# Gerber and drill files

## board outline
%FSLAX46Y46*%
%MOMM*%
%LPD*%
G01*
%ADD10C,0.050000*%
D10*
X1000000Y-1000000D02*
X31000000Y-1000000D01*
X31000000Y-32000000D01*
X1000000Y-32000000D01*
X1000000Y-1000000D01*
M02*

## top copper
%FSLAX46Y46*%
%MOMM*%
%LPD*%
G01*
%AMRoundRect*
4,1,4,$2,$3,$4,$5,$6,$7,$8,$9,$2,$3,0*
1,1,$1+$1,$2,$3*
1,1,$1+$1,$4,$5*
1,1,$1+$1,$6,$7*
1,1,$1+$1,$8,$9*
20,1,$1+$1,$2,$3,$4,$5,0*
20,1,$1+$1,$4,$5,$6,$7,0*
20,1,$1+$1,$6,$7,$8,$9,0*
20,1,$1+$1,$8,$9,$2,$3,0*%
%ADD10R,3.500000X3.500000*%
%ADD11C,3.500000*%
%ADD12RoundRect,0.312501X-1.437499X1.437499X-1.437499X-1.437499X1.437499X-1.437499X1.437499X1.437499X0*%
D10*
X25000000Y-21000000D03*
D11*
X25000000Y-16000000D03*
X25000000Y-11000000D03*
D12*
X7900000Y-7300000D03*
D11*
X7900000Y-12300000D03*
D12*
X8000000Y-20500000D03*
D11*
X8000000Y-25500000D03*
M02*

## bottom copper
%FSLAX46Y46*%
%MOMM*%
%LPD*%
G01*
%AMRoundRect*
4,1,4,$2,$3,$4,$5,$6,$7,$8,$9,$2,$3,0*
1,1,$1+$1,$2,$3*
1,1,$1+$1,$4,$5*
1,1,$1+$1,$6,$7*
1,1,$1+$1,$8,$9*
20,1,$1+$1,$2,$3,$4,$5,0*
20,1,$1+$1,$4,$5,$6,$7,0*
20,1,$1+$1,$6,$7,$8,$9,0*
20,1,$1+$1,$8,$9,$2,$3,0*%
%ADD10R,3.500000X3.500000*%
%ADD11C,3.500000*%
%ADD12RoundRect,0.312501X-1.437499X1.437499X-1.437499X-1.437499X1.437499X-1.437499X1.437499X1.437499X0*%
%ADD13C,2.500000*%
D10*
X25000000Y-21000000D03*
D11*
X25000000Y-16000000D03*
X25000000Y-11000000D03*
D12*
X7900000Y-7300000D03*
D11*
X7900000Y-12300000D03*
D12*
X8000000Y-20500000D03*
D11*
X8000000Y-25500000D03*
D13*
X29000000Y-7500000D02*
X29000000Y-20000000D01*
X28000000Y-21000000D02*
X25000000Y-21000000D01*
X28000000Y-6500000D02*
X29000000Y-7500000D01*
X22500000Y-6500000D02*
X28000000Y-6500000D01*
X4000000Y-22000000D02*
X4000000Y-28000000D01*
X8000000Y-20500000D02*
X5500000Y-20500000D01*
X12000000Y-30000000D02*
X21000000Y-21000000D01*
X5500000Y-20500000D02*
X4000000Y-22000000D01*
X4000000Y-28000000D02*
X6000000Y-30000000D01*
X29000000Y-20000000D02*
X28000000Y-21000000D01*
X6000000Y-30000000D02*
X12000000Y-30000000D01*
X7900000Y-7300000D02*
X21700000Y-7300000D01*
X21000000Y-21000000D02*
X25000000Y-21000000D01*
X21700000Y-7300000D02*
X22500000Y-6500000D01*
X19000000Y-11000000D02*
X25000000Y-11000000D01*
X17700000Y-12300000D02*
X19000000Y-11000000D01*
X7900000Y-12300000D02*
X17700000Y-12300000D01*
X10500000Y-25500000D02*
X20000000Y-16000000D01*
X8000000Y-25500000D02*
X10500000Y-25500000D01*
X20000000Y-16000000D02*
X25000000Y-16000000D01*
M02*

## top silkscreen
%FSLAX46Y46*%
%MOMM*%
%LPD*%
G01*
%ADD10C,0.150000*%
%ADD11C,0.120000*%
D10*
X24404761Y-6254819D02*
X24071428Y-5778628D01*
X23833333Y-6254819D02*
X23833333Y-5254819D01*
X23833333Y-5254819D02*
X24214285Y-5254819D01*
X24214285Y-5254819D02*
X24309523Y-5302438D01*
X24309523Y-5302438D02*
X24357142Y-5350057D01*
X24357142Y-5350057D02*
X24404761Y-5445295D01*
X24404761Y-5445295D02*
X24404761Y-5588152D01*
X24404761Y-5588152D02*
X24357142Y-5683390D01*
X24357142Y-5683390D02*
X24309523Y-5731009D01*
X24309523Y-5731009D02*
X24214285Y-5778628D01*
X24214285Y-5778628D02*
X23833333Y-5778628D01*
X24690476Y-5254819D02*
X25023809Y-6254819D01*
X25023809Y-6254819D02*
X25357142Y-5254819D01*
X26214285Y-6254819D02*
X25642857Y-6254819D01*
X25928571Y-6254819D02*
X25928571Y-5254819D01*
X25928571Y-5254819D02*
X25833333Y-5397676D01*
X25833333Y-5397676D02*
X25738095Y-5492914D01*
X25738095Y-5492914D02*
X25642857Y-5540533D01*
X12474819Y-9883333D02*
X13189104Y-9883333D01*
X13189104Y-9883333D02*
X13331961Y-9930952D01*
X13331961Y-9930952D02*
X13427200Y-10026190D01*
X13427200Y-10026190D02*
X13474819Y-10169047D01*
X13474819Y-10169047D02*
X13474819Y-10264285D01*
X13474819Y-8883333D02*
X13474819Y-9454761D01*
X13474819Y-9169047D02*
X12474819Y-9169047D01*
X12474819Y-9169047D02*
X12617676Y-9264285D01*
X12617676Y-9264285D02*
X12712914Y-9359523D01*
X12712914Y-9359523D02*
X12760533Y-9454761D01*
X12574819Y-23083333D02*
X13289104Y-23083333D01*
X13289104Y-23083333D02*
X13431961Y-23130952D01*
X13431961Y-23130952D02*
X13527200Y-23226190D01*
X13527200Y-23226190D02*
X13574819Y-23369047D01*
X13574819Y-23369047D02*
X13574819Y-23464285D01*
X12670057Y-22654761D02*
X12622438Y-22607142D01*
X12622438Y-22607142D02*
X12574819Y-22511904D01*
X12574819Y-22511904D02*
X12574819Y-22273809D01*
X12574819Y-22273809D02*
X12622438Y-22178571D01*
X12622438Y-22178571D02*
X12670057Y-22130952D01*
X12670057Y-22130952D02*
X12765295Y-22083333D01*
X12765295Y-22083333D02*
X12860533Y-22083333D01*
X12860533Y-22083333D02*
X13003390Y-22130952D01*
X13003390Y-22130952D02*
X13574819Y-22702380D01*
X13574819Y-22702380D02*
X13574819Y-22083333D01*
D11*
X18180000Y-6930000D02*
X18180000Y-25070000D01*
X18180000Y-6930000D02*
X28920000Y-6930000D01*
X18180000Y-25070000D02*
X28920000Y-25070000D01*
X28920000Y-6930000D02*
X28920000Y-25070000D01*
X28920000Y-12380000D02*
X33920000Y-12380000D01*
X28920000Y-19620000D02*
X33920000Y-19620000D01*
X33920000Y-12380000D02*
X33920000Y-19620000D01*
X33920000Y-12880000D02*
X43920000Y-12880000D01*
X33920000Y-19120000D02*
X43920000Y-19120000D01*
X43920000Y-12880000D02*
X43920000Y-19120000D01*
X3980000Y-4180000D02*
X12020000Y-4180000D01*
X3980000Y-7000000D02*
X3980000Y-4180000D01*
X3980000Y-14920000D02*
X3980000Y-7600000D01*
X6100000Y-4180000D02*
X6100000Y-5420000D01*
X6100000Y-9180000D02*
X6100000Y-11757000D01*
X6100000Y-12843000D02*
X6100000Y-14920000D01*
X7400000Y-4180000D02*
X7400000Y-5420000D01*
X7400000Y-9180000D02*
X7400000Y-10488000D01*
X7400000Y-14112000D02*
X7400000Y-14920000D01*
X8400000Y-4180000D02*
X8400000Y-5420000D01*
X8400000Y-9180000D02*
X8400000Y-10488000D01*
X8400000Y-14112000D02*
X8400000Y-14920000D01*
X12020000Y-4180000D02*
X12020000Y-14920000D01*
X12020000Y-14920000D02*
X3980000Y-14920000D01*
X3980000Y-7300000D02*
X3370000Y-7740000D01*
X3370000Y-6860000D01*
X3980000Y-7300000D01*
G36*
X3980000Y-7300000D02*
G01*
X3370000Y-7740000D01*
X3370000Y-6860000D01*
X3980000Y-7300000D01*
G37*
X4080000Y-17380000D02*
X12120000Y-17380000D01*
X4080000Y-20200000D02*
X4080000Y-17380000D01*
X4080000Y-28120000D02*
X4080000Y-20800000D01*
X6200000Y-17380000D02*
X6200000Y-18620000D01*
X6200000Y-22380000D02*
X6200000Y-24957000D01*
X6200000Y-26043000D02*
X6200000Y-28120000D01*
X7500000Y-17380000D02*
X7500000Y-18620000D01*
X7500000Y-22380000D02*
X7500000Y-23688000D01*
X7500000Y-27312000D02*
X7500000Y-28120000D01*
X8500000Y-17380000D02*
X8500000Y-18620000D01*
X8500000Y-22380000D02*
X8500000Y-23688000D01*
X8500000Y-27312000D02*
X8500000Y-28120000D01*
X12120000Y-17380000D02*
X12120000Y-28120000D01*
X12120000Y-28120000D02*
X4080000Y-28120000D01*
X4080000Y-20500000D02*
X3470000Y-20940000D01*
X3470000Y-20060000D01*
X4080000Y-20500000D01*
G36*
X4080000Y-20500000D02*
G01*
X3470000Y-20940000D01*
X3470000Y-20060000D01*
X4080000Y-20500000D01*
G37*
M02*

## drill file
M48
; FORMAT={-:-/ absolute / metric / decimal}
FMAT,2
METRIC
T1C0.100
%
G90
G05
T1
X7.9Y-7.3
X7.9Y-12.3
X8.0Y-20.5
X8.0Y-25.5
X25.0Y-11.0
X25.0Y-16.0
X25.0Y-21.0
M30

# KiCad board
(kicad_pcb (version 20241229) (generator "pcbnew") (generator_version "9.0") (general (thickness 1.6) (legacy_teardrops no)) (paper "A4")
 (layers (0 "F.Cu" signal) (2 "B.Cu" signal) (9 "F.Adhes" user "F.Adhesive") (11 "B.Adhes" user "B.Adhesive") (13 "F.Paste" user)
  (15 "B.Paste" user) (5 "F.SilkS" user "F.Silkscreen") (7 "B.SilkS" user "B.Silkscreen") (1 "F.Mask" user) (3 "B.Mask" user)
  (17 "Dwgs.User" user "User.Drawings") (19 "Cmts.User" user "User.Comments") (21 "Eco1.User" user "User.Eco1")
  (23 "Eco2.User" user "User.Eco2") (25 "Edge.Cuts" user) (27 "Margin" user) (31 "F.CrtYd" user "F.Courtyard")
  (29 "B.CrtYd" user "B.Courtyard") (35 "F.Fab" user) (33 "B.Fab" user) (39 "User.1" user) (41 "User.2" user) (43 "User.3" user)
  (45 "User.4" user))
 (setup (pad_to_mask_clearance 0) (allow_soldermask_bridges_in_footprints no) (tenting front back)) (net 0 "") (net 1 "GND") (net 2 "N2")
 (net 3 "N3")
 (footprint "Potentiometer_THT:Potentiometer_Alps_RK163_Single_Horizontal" (layer "F.Cu") (at 25 21 180)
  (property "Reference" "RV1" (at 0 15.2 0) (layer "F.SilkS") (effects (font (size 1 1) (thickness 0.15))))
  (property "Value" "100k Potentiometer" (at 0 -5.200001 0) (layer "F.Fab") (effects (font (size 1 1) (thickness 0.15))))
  (fp_line (start 6.82 14.07) (end 6.82 -4.07) (stroke (width 0.12) (type solid)) (layer "F.SilkS"))
  (fp_line (start 6.82 14.07) (end -3.92 14.07) (stroke (width 0.12) (type solid)) (layer "F.SilkS"))
  (fp_line (start 6.82 -4.07) (end -3.92 -4.07) (stroke (width 0.12) (type solid)) (layer "F.SilkS"))
  (fp_line (start -3.92 14.07) (end -3.92 -4.07) (stroke (width 0.12) (type solid)) (layer "F.SilkS"))
  (fp_line (start -3.92 8.62) (end -8.92 8.62) (stroke (width 0.12) (type solid)) (layer "F.SilkS"))
  (fp_line (start -3.92 1.38) (end -8.92 1.38) (stroke (width 0.12) (type solid)) (layer "F.SilkS"))
  (fp_line (start -8.92 8.62) (end -8.92 1.38) (stroke (width 0.12) (type solid)) (layer "F.SilkS"))
  (fp_line (start -8.92 8.12) (end -18.92 8.12) (stroke (width 0.12) (type solid)) (layer "F.SilkS"))
  (fp_line (start -8.92 1.88) (end -18.92 1.88) (stroke (width 0.12) (type solid)) (layer "F.SilkS"))
  (fp_line (start -18.92 8.12) (end -18.92 1.88) (stroke (width 0.12) (type solid)) (layer "F.SilkS"))
  (pad "1" thru_hole rect (at 0 0) (size 3.5 3.5) (drill 0.1) (layers "*.Cu" "*.Mask") (remove_unused_layers no) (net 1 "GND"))
  (pad "2" thru_hole circle (at 0 5) (size 3.5 3.5) (drill 0.1) (layers "*.Cu" "*.Mask") (remove_unused_layers no) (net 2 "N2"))
  (pad "3" thru_hole circle (at 0 10) (size 3.5 3.5) (drill 0.1) (layers "*.Cu" "*.Mask") (remove_unused_layers no) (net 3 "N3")))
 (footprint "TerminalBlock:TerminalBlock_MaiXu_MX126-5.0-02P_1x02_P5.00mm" (layer "F.Cu") (at 7.9 7.3 -90)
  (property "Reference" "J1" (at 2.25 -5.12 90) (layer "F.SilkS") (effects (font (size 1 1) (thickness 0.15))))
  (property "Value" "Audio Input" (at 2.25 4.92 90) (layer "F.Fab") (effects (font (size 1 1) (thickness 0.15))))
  (fp_line (start -3.12 3.92) (end -3.12 -4.12) (stroke (width 0.12) (type solid)) (layer "F.SilkS"))
  (fp_line (start -0.3 3.92) (end -3.12 3.92) (stroke (width 0.12) (type solid)) (layer "F.SilkS"))
  (fp_line (start 7.62 3.92) (end 0.3 3.92) (stroke (width 0.12) (type solid)) (layer "F.SilkS"))
  (fp_line (start -3.12 1.8) (end -1.88 1.8) (stroke (width 0.12) (type solid)) (layer "F.SilkS"))
  (fp_line (start 1.88 1.8) (end 4.457 1.8) (stroke (width 0.12) (type solid)) (layer "F.SilkS"))
  (fp_line (start 5.543 1.8) (end 7.62 1.8) (stroke (width 0.12) (type solid)) (layer "F.SilkS"))
  (fp_line (start -3.12 0.5) (end -1.88 0.5) (stroke (width 0.12) (type solid)) (layer "F.SilkS"))
  (fp_line (start 1.88 0.5) (end 3.188 0.5) (stroke (width 0.12) (type solid)) (layer "F.SilkS"))
  (fp_line (start 6.812 0.5) (end 7.62 0.5) (stroke (width 0.12) (type solid)) (layer "F.SilkS"))
  (fp_line (start -3.12 -0.5) (end -1.88 -0.5) (stroke (width 0.12) (type solid)) (layer "F.SilkS"))
  (fp_line (start 1.88 -0.5) (end 3.188 -0.5) (stroke (width 0.12) (type solid)) (layer "F.SilkS"))
  (fp_line (start 6.812 -0.5) (end 7.62 -0.5) (stroke (width 0.12) (type solid)) (layer "F.SilkS"))
  (fp_line (start -3.12 -4.12) (end 7.62 -4.12) (stroke (width 0.12) (type solid)) (layer "F.SilkS"))
  (fp_line (start 7.62 -4.12) (end 7.62 3.92) (stroke (width 0.12) (type solid)) (layer "F.SilkS"))
  (fp_poly (pts (xy 0 3.92) (xy 0.44 4.53) (xy -0.44 4.53)) (stroke (width 0.12) (type solid)) (fill yes) (layer "F.SilkS"))
  (pad "1" thru_hole roundrect (at 0 0 270) (size 3.5 3.5) (drill 0.1) (layers "*.Cu" "*.Mask") (remove_unused_layers no)
   (roundrect_rratio 0.089286) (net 1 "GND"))
  (pad "2" thru_hole circle (at 5 0 270) (size 3.5 3.5) (drill 0.1) (layers "*.Cu" "*.Mask") (remove_unused_layers no) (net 3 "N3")))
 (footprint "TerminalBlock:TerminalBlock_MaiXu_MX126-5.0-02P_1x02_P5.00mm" (layer "F.Cu") (at 8 20.5 -90)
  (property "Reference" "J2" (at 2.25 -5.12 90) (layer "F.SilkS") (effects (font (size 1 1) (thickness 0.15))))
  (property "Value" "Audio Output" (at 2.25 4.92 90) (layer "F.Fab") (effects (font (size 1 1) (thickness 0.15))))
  (fp_line (start -3.12 3.92) (end -3.12 -4.12) (stroke (width 0.12) (type solid)) (layer "F.SilkS"))
  (fp_line (start -0.3 3.92) (end -3.12 3.92) (stroke (width 0.12) (type solid)) (layer "F.SilkS"))
  (fp_line (start 7.62 3.92) (end 0.3 3.92) (stroke (width 0.12) (type solid)) (layer "F.SilkS"))
  (fp_line (start -3.12 1.8) (end -1.88 1.8) (stroke (width 0.12) (type solid)) (layer "F.SilkS"))
  (fp_line (start 1.88 1.8) (end 4.457 1.8) (stroke (width 0.12) (type solid)) (layer "F.SilkS"))
  (fp_line (start 5.543 1.8) (end 7.62 1.8) (stroke (width 0.12) (type solid)) (layer "F.SilkS"))
  (fp_line (start -3.12 0.5) (end -1.88 0.5) (stroke (width 0.12) (type solid)) (layer "F.SilkS"))
  (fp_line (start 1.88 0.5) (end 3.188 0.5) (stroke (width 0.12) (type solid)) (layer "F.SilkS"))
  (fp_line (start 6.812 0.5) (end 7.62 0.5) (stroke (width 0.12) (type solid)) (layer "F.SilkS"))
  (fp_line (start -3.12 -0.5) (end -1.88 -0.5) (stroke (width 0.12) (type solid)) (layer "F.SilkS"))
  (fp_line (start 1.88 -0.5) (end 3.188 -0.5) (stroke (width 0.12) (type solid)) (layer "F.SilkS"))
  (fp_line (start 6.812 -0.5) (end 7.62 -0.5) (stroke (width 0.12) (type solid)) (layer "F.SilkS"))
  (fp_line (start -3.12 -4.12) (end 7.62 -4.12) (stroke (width 0.12) (type solid)) (layer "F.SilkS"))
  (fp_line (start 7.62 -4.12) (end 7.62 3.92) (stroke (width 0.12) (type solid)) (layer "F.SilkS"))
  (fp_poly (pts (xy 0 3.92) (xy 0.44 4.53) (xy -0.44 4.53)) (stroke (width 0.12) (type solid)) (fill yes) (layer "F.SilkS"))
  (pad "1" thru_hole roundrect (at 0 0 270) (size 3.5 3.5) (drill 0.1) (layers "*.Cu" "*.Mask") (remove_unused_layers no)
   (roundrect_rratio 0.089286) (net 1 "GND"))
  (pad "2" thru_hole circle (at 5 0 270) (size 3.5 3.5) (drill 0.1) (layers "*.Cu" "*.Mask") (remove_unused_layers no) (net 2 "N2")))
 (gr_rect (start 1 1) (end 31 32) (stroke (width 0.05) (type default)) (fill no) (layer "Edge.Cuts"))
 (segment (start 29 7.5) (end 29 20) (width 2.5) (layer "B.Cu") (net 1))
 (segment (start 28 21) (end 25 21) (width 2.5) (layer "B.Cu") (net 1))
 (segment (start 28 6.5) (end 29 7.5) (width 2.5) (layer "B.Cu") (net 1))
 (segment (start 22.5 6.5) (end 28 6.5) (width 2.5) (layer "B.Cu") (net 1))
 (segment (start 4 22) (end 4 28) (width 2.5) (layer "B.Cu") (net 1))
 (segment (start 8 20.5) (end 5.5 20.5) (width 2.5) (layer "B.Cu") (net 1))
 (segment (start 12 30) (end 21 21) (width 2.5) (layer "B.Cu") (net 1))
 (segment (start 5.5 20.5) (end 4 22) (width 2.5) (layer "B.Cu") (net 1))
 (segment (start 4 28) (end 6 30) (width 2.5) (layer "B.Cu") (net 1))
 (segment (start 29 20) (end 28 21) (width 2.5) (layer "B.Cu") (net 1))
 (segment (start 6 30) (end 12 30) (width 2.5) (layer "B.Cu") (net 1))
 (segment (start 7.9 7.3) (end 21.7 7.3) (width 2.5) (layer "B.Cu") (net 1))
 (segment (start 21 21) (end 25 21) (width 2.5) (layer "B.Cu") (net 1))
 (segment (start 21.7 7.3) (end 22.5 6.5) (width 2.5) (layer "B.Cu") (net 1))
 (segment (start 19 11) (end 25 11) (width 2.5) (layer "B.Cu") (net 3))
 (segment (start 17.7 12.3) (end 19 11) (width 2.5) (layer "B.Cu") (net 3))
 (segment (start 7.9 12.3) (end 17.7 12.3) (width 2.5) (layer "B.Cu") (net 3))
 (segment (start 10.5 25.5) (end 20 16) (width 2.5) (layer "B.Cu") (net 2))
 (segment (start 8 25.5) (end 10.5 25.5) (width 2.5) (layer "B.Cu") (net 2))
 (segment (start 20 16) (end 25 16) (width 2.5) (layer "B.Cu") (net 2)))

